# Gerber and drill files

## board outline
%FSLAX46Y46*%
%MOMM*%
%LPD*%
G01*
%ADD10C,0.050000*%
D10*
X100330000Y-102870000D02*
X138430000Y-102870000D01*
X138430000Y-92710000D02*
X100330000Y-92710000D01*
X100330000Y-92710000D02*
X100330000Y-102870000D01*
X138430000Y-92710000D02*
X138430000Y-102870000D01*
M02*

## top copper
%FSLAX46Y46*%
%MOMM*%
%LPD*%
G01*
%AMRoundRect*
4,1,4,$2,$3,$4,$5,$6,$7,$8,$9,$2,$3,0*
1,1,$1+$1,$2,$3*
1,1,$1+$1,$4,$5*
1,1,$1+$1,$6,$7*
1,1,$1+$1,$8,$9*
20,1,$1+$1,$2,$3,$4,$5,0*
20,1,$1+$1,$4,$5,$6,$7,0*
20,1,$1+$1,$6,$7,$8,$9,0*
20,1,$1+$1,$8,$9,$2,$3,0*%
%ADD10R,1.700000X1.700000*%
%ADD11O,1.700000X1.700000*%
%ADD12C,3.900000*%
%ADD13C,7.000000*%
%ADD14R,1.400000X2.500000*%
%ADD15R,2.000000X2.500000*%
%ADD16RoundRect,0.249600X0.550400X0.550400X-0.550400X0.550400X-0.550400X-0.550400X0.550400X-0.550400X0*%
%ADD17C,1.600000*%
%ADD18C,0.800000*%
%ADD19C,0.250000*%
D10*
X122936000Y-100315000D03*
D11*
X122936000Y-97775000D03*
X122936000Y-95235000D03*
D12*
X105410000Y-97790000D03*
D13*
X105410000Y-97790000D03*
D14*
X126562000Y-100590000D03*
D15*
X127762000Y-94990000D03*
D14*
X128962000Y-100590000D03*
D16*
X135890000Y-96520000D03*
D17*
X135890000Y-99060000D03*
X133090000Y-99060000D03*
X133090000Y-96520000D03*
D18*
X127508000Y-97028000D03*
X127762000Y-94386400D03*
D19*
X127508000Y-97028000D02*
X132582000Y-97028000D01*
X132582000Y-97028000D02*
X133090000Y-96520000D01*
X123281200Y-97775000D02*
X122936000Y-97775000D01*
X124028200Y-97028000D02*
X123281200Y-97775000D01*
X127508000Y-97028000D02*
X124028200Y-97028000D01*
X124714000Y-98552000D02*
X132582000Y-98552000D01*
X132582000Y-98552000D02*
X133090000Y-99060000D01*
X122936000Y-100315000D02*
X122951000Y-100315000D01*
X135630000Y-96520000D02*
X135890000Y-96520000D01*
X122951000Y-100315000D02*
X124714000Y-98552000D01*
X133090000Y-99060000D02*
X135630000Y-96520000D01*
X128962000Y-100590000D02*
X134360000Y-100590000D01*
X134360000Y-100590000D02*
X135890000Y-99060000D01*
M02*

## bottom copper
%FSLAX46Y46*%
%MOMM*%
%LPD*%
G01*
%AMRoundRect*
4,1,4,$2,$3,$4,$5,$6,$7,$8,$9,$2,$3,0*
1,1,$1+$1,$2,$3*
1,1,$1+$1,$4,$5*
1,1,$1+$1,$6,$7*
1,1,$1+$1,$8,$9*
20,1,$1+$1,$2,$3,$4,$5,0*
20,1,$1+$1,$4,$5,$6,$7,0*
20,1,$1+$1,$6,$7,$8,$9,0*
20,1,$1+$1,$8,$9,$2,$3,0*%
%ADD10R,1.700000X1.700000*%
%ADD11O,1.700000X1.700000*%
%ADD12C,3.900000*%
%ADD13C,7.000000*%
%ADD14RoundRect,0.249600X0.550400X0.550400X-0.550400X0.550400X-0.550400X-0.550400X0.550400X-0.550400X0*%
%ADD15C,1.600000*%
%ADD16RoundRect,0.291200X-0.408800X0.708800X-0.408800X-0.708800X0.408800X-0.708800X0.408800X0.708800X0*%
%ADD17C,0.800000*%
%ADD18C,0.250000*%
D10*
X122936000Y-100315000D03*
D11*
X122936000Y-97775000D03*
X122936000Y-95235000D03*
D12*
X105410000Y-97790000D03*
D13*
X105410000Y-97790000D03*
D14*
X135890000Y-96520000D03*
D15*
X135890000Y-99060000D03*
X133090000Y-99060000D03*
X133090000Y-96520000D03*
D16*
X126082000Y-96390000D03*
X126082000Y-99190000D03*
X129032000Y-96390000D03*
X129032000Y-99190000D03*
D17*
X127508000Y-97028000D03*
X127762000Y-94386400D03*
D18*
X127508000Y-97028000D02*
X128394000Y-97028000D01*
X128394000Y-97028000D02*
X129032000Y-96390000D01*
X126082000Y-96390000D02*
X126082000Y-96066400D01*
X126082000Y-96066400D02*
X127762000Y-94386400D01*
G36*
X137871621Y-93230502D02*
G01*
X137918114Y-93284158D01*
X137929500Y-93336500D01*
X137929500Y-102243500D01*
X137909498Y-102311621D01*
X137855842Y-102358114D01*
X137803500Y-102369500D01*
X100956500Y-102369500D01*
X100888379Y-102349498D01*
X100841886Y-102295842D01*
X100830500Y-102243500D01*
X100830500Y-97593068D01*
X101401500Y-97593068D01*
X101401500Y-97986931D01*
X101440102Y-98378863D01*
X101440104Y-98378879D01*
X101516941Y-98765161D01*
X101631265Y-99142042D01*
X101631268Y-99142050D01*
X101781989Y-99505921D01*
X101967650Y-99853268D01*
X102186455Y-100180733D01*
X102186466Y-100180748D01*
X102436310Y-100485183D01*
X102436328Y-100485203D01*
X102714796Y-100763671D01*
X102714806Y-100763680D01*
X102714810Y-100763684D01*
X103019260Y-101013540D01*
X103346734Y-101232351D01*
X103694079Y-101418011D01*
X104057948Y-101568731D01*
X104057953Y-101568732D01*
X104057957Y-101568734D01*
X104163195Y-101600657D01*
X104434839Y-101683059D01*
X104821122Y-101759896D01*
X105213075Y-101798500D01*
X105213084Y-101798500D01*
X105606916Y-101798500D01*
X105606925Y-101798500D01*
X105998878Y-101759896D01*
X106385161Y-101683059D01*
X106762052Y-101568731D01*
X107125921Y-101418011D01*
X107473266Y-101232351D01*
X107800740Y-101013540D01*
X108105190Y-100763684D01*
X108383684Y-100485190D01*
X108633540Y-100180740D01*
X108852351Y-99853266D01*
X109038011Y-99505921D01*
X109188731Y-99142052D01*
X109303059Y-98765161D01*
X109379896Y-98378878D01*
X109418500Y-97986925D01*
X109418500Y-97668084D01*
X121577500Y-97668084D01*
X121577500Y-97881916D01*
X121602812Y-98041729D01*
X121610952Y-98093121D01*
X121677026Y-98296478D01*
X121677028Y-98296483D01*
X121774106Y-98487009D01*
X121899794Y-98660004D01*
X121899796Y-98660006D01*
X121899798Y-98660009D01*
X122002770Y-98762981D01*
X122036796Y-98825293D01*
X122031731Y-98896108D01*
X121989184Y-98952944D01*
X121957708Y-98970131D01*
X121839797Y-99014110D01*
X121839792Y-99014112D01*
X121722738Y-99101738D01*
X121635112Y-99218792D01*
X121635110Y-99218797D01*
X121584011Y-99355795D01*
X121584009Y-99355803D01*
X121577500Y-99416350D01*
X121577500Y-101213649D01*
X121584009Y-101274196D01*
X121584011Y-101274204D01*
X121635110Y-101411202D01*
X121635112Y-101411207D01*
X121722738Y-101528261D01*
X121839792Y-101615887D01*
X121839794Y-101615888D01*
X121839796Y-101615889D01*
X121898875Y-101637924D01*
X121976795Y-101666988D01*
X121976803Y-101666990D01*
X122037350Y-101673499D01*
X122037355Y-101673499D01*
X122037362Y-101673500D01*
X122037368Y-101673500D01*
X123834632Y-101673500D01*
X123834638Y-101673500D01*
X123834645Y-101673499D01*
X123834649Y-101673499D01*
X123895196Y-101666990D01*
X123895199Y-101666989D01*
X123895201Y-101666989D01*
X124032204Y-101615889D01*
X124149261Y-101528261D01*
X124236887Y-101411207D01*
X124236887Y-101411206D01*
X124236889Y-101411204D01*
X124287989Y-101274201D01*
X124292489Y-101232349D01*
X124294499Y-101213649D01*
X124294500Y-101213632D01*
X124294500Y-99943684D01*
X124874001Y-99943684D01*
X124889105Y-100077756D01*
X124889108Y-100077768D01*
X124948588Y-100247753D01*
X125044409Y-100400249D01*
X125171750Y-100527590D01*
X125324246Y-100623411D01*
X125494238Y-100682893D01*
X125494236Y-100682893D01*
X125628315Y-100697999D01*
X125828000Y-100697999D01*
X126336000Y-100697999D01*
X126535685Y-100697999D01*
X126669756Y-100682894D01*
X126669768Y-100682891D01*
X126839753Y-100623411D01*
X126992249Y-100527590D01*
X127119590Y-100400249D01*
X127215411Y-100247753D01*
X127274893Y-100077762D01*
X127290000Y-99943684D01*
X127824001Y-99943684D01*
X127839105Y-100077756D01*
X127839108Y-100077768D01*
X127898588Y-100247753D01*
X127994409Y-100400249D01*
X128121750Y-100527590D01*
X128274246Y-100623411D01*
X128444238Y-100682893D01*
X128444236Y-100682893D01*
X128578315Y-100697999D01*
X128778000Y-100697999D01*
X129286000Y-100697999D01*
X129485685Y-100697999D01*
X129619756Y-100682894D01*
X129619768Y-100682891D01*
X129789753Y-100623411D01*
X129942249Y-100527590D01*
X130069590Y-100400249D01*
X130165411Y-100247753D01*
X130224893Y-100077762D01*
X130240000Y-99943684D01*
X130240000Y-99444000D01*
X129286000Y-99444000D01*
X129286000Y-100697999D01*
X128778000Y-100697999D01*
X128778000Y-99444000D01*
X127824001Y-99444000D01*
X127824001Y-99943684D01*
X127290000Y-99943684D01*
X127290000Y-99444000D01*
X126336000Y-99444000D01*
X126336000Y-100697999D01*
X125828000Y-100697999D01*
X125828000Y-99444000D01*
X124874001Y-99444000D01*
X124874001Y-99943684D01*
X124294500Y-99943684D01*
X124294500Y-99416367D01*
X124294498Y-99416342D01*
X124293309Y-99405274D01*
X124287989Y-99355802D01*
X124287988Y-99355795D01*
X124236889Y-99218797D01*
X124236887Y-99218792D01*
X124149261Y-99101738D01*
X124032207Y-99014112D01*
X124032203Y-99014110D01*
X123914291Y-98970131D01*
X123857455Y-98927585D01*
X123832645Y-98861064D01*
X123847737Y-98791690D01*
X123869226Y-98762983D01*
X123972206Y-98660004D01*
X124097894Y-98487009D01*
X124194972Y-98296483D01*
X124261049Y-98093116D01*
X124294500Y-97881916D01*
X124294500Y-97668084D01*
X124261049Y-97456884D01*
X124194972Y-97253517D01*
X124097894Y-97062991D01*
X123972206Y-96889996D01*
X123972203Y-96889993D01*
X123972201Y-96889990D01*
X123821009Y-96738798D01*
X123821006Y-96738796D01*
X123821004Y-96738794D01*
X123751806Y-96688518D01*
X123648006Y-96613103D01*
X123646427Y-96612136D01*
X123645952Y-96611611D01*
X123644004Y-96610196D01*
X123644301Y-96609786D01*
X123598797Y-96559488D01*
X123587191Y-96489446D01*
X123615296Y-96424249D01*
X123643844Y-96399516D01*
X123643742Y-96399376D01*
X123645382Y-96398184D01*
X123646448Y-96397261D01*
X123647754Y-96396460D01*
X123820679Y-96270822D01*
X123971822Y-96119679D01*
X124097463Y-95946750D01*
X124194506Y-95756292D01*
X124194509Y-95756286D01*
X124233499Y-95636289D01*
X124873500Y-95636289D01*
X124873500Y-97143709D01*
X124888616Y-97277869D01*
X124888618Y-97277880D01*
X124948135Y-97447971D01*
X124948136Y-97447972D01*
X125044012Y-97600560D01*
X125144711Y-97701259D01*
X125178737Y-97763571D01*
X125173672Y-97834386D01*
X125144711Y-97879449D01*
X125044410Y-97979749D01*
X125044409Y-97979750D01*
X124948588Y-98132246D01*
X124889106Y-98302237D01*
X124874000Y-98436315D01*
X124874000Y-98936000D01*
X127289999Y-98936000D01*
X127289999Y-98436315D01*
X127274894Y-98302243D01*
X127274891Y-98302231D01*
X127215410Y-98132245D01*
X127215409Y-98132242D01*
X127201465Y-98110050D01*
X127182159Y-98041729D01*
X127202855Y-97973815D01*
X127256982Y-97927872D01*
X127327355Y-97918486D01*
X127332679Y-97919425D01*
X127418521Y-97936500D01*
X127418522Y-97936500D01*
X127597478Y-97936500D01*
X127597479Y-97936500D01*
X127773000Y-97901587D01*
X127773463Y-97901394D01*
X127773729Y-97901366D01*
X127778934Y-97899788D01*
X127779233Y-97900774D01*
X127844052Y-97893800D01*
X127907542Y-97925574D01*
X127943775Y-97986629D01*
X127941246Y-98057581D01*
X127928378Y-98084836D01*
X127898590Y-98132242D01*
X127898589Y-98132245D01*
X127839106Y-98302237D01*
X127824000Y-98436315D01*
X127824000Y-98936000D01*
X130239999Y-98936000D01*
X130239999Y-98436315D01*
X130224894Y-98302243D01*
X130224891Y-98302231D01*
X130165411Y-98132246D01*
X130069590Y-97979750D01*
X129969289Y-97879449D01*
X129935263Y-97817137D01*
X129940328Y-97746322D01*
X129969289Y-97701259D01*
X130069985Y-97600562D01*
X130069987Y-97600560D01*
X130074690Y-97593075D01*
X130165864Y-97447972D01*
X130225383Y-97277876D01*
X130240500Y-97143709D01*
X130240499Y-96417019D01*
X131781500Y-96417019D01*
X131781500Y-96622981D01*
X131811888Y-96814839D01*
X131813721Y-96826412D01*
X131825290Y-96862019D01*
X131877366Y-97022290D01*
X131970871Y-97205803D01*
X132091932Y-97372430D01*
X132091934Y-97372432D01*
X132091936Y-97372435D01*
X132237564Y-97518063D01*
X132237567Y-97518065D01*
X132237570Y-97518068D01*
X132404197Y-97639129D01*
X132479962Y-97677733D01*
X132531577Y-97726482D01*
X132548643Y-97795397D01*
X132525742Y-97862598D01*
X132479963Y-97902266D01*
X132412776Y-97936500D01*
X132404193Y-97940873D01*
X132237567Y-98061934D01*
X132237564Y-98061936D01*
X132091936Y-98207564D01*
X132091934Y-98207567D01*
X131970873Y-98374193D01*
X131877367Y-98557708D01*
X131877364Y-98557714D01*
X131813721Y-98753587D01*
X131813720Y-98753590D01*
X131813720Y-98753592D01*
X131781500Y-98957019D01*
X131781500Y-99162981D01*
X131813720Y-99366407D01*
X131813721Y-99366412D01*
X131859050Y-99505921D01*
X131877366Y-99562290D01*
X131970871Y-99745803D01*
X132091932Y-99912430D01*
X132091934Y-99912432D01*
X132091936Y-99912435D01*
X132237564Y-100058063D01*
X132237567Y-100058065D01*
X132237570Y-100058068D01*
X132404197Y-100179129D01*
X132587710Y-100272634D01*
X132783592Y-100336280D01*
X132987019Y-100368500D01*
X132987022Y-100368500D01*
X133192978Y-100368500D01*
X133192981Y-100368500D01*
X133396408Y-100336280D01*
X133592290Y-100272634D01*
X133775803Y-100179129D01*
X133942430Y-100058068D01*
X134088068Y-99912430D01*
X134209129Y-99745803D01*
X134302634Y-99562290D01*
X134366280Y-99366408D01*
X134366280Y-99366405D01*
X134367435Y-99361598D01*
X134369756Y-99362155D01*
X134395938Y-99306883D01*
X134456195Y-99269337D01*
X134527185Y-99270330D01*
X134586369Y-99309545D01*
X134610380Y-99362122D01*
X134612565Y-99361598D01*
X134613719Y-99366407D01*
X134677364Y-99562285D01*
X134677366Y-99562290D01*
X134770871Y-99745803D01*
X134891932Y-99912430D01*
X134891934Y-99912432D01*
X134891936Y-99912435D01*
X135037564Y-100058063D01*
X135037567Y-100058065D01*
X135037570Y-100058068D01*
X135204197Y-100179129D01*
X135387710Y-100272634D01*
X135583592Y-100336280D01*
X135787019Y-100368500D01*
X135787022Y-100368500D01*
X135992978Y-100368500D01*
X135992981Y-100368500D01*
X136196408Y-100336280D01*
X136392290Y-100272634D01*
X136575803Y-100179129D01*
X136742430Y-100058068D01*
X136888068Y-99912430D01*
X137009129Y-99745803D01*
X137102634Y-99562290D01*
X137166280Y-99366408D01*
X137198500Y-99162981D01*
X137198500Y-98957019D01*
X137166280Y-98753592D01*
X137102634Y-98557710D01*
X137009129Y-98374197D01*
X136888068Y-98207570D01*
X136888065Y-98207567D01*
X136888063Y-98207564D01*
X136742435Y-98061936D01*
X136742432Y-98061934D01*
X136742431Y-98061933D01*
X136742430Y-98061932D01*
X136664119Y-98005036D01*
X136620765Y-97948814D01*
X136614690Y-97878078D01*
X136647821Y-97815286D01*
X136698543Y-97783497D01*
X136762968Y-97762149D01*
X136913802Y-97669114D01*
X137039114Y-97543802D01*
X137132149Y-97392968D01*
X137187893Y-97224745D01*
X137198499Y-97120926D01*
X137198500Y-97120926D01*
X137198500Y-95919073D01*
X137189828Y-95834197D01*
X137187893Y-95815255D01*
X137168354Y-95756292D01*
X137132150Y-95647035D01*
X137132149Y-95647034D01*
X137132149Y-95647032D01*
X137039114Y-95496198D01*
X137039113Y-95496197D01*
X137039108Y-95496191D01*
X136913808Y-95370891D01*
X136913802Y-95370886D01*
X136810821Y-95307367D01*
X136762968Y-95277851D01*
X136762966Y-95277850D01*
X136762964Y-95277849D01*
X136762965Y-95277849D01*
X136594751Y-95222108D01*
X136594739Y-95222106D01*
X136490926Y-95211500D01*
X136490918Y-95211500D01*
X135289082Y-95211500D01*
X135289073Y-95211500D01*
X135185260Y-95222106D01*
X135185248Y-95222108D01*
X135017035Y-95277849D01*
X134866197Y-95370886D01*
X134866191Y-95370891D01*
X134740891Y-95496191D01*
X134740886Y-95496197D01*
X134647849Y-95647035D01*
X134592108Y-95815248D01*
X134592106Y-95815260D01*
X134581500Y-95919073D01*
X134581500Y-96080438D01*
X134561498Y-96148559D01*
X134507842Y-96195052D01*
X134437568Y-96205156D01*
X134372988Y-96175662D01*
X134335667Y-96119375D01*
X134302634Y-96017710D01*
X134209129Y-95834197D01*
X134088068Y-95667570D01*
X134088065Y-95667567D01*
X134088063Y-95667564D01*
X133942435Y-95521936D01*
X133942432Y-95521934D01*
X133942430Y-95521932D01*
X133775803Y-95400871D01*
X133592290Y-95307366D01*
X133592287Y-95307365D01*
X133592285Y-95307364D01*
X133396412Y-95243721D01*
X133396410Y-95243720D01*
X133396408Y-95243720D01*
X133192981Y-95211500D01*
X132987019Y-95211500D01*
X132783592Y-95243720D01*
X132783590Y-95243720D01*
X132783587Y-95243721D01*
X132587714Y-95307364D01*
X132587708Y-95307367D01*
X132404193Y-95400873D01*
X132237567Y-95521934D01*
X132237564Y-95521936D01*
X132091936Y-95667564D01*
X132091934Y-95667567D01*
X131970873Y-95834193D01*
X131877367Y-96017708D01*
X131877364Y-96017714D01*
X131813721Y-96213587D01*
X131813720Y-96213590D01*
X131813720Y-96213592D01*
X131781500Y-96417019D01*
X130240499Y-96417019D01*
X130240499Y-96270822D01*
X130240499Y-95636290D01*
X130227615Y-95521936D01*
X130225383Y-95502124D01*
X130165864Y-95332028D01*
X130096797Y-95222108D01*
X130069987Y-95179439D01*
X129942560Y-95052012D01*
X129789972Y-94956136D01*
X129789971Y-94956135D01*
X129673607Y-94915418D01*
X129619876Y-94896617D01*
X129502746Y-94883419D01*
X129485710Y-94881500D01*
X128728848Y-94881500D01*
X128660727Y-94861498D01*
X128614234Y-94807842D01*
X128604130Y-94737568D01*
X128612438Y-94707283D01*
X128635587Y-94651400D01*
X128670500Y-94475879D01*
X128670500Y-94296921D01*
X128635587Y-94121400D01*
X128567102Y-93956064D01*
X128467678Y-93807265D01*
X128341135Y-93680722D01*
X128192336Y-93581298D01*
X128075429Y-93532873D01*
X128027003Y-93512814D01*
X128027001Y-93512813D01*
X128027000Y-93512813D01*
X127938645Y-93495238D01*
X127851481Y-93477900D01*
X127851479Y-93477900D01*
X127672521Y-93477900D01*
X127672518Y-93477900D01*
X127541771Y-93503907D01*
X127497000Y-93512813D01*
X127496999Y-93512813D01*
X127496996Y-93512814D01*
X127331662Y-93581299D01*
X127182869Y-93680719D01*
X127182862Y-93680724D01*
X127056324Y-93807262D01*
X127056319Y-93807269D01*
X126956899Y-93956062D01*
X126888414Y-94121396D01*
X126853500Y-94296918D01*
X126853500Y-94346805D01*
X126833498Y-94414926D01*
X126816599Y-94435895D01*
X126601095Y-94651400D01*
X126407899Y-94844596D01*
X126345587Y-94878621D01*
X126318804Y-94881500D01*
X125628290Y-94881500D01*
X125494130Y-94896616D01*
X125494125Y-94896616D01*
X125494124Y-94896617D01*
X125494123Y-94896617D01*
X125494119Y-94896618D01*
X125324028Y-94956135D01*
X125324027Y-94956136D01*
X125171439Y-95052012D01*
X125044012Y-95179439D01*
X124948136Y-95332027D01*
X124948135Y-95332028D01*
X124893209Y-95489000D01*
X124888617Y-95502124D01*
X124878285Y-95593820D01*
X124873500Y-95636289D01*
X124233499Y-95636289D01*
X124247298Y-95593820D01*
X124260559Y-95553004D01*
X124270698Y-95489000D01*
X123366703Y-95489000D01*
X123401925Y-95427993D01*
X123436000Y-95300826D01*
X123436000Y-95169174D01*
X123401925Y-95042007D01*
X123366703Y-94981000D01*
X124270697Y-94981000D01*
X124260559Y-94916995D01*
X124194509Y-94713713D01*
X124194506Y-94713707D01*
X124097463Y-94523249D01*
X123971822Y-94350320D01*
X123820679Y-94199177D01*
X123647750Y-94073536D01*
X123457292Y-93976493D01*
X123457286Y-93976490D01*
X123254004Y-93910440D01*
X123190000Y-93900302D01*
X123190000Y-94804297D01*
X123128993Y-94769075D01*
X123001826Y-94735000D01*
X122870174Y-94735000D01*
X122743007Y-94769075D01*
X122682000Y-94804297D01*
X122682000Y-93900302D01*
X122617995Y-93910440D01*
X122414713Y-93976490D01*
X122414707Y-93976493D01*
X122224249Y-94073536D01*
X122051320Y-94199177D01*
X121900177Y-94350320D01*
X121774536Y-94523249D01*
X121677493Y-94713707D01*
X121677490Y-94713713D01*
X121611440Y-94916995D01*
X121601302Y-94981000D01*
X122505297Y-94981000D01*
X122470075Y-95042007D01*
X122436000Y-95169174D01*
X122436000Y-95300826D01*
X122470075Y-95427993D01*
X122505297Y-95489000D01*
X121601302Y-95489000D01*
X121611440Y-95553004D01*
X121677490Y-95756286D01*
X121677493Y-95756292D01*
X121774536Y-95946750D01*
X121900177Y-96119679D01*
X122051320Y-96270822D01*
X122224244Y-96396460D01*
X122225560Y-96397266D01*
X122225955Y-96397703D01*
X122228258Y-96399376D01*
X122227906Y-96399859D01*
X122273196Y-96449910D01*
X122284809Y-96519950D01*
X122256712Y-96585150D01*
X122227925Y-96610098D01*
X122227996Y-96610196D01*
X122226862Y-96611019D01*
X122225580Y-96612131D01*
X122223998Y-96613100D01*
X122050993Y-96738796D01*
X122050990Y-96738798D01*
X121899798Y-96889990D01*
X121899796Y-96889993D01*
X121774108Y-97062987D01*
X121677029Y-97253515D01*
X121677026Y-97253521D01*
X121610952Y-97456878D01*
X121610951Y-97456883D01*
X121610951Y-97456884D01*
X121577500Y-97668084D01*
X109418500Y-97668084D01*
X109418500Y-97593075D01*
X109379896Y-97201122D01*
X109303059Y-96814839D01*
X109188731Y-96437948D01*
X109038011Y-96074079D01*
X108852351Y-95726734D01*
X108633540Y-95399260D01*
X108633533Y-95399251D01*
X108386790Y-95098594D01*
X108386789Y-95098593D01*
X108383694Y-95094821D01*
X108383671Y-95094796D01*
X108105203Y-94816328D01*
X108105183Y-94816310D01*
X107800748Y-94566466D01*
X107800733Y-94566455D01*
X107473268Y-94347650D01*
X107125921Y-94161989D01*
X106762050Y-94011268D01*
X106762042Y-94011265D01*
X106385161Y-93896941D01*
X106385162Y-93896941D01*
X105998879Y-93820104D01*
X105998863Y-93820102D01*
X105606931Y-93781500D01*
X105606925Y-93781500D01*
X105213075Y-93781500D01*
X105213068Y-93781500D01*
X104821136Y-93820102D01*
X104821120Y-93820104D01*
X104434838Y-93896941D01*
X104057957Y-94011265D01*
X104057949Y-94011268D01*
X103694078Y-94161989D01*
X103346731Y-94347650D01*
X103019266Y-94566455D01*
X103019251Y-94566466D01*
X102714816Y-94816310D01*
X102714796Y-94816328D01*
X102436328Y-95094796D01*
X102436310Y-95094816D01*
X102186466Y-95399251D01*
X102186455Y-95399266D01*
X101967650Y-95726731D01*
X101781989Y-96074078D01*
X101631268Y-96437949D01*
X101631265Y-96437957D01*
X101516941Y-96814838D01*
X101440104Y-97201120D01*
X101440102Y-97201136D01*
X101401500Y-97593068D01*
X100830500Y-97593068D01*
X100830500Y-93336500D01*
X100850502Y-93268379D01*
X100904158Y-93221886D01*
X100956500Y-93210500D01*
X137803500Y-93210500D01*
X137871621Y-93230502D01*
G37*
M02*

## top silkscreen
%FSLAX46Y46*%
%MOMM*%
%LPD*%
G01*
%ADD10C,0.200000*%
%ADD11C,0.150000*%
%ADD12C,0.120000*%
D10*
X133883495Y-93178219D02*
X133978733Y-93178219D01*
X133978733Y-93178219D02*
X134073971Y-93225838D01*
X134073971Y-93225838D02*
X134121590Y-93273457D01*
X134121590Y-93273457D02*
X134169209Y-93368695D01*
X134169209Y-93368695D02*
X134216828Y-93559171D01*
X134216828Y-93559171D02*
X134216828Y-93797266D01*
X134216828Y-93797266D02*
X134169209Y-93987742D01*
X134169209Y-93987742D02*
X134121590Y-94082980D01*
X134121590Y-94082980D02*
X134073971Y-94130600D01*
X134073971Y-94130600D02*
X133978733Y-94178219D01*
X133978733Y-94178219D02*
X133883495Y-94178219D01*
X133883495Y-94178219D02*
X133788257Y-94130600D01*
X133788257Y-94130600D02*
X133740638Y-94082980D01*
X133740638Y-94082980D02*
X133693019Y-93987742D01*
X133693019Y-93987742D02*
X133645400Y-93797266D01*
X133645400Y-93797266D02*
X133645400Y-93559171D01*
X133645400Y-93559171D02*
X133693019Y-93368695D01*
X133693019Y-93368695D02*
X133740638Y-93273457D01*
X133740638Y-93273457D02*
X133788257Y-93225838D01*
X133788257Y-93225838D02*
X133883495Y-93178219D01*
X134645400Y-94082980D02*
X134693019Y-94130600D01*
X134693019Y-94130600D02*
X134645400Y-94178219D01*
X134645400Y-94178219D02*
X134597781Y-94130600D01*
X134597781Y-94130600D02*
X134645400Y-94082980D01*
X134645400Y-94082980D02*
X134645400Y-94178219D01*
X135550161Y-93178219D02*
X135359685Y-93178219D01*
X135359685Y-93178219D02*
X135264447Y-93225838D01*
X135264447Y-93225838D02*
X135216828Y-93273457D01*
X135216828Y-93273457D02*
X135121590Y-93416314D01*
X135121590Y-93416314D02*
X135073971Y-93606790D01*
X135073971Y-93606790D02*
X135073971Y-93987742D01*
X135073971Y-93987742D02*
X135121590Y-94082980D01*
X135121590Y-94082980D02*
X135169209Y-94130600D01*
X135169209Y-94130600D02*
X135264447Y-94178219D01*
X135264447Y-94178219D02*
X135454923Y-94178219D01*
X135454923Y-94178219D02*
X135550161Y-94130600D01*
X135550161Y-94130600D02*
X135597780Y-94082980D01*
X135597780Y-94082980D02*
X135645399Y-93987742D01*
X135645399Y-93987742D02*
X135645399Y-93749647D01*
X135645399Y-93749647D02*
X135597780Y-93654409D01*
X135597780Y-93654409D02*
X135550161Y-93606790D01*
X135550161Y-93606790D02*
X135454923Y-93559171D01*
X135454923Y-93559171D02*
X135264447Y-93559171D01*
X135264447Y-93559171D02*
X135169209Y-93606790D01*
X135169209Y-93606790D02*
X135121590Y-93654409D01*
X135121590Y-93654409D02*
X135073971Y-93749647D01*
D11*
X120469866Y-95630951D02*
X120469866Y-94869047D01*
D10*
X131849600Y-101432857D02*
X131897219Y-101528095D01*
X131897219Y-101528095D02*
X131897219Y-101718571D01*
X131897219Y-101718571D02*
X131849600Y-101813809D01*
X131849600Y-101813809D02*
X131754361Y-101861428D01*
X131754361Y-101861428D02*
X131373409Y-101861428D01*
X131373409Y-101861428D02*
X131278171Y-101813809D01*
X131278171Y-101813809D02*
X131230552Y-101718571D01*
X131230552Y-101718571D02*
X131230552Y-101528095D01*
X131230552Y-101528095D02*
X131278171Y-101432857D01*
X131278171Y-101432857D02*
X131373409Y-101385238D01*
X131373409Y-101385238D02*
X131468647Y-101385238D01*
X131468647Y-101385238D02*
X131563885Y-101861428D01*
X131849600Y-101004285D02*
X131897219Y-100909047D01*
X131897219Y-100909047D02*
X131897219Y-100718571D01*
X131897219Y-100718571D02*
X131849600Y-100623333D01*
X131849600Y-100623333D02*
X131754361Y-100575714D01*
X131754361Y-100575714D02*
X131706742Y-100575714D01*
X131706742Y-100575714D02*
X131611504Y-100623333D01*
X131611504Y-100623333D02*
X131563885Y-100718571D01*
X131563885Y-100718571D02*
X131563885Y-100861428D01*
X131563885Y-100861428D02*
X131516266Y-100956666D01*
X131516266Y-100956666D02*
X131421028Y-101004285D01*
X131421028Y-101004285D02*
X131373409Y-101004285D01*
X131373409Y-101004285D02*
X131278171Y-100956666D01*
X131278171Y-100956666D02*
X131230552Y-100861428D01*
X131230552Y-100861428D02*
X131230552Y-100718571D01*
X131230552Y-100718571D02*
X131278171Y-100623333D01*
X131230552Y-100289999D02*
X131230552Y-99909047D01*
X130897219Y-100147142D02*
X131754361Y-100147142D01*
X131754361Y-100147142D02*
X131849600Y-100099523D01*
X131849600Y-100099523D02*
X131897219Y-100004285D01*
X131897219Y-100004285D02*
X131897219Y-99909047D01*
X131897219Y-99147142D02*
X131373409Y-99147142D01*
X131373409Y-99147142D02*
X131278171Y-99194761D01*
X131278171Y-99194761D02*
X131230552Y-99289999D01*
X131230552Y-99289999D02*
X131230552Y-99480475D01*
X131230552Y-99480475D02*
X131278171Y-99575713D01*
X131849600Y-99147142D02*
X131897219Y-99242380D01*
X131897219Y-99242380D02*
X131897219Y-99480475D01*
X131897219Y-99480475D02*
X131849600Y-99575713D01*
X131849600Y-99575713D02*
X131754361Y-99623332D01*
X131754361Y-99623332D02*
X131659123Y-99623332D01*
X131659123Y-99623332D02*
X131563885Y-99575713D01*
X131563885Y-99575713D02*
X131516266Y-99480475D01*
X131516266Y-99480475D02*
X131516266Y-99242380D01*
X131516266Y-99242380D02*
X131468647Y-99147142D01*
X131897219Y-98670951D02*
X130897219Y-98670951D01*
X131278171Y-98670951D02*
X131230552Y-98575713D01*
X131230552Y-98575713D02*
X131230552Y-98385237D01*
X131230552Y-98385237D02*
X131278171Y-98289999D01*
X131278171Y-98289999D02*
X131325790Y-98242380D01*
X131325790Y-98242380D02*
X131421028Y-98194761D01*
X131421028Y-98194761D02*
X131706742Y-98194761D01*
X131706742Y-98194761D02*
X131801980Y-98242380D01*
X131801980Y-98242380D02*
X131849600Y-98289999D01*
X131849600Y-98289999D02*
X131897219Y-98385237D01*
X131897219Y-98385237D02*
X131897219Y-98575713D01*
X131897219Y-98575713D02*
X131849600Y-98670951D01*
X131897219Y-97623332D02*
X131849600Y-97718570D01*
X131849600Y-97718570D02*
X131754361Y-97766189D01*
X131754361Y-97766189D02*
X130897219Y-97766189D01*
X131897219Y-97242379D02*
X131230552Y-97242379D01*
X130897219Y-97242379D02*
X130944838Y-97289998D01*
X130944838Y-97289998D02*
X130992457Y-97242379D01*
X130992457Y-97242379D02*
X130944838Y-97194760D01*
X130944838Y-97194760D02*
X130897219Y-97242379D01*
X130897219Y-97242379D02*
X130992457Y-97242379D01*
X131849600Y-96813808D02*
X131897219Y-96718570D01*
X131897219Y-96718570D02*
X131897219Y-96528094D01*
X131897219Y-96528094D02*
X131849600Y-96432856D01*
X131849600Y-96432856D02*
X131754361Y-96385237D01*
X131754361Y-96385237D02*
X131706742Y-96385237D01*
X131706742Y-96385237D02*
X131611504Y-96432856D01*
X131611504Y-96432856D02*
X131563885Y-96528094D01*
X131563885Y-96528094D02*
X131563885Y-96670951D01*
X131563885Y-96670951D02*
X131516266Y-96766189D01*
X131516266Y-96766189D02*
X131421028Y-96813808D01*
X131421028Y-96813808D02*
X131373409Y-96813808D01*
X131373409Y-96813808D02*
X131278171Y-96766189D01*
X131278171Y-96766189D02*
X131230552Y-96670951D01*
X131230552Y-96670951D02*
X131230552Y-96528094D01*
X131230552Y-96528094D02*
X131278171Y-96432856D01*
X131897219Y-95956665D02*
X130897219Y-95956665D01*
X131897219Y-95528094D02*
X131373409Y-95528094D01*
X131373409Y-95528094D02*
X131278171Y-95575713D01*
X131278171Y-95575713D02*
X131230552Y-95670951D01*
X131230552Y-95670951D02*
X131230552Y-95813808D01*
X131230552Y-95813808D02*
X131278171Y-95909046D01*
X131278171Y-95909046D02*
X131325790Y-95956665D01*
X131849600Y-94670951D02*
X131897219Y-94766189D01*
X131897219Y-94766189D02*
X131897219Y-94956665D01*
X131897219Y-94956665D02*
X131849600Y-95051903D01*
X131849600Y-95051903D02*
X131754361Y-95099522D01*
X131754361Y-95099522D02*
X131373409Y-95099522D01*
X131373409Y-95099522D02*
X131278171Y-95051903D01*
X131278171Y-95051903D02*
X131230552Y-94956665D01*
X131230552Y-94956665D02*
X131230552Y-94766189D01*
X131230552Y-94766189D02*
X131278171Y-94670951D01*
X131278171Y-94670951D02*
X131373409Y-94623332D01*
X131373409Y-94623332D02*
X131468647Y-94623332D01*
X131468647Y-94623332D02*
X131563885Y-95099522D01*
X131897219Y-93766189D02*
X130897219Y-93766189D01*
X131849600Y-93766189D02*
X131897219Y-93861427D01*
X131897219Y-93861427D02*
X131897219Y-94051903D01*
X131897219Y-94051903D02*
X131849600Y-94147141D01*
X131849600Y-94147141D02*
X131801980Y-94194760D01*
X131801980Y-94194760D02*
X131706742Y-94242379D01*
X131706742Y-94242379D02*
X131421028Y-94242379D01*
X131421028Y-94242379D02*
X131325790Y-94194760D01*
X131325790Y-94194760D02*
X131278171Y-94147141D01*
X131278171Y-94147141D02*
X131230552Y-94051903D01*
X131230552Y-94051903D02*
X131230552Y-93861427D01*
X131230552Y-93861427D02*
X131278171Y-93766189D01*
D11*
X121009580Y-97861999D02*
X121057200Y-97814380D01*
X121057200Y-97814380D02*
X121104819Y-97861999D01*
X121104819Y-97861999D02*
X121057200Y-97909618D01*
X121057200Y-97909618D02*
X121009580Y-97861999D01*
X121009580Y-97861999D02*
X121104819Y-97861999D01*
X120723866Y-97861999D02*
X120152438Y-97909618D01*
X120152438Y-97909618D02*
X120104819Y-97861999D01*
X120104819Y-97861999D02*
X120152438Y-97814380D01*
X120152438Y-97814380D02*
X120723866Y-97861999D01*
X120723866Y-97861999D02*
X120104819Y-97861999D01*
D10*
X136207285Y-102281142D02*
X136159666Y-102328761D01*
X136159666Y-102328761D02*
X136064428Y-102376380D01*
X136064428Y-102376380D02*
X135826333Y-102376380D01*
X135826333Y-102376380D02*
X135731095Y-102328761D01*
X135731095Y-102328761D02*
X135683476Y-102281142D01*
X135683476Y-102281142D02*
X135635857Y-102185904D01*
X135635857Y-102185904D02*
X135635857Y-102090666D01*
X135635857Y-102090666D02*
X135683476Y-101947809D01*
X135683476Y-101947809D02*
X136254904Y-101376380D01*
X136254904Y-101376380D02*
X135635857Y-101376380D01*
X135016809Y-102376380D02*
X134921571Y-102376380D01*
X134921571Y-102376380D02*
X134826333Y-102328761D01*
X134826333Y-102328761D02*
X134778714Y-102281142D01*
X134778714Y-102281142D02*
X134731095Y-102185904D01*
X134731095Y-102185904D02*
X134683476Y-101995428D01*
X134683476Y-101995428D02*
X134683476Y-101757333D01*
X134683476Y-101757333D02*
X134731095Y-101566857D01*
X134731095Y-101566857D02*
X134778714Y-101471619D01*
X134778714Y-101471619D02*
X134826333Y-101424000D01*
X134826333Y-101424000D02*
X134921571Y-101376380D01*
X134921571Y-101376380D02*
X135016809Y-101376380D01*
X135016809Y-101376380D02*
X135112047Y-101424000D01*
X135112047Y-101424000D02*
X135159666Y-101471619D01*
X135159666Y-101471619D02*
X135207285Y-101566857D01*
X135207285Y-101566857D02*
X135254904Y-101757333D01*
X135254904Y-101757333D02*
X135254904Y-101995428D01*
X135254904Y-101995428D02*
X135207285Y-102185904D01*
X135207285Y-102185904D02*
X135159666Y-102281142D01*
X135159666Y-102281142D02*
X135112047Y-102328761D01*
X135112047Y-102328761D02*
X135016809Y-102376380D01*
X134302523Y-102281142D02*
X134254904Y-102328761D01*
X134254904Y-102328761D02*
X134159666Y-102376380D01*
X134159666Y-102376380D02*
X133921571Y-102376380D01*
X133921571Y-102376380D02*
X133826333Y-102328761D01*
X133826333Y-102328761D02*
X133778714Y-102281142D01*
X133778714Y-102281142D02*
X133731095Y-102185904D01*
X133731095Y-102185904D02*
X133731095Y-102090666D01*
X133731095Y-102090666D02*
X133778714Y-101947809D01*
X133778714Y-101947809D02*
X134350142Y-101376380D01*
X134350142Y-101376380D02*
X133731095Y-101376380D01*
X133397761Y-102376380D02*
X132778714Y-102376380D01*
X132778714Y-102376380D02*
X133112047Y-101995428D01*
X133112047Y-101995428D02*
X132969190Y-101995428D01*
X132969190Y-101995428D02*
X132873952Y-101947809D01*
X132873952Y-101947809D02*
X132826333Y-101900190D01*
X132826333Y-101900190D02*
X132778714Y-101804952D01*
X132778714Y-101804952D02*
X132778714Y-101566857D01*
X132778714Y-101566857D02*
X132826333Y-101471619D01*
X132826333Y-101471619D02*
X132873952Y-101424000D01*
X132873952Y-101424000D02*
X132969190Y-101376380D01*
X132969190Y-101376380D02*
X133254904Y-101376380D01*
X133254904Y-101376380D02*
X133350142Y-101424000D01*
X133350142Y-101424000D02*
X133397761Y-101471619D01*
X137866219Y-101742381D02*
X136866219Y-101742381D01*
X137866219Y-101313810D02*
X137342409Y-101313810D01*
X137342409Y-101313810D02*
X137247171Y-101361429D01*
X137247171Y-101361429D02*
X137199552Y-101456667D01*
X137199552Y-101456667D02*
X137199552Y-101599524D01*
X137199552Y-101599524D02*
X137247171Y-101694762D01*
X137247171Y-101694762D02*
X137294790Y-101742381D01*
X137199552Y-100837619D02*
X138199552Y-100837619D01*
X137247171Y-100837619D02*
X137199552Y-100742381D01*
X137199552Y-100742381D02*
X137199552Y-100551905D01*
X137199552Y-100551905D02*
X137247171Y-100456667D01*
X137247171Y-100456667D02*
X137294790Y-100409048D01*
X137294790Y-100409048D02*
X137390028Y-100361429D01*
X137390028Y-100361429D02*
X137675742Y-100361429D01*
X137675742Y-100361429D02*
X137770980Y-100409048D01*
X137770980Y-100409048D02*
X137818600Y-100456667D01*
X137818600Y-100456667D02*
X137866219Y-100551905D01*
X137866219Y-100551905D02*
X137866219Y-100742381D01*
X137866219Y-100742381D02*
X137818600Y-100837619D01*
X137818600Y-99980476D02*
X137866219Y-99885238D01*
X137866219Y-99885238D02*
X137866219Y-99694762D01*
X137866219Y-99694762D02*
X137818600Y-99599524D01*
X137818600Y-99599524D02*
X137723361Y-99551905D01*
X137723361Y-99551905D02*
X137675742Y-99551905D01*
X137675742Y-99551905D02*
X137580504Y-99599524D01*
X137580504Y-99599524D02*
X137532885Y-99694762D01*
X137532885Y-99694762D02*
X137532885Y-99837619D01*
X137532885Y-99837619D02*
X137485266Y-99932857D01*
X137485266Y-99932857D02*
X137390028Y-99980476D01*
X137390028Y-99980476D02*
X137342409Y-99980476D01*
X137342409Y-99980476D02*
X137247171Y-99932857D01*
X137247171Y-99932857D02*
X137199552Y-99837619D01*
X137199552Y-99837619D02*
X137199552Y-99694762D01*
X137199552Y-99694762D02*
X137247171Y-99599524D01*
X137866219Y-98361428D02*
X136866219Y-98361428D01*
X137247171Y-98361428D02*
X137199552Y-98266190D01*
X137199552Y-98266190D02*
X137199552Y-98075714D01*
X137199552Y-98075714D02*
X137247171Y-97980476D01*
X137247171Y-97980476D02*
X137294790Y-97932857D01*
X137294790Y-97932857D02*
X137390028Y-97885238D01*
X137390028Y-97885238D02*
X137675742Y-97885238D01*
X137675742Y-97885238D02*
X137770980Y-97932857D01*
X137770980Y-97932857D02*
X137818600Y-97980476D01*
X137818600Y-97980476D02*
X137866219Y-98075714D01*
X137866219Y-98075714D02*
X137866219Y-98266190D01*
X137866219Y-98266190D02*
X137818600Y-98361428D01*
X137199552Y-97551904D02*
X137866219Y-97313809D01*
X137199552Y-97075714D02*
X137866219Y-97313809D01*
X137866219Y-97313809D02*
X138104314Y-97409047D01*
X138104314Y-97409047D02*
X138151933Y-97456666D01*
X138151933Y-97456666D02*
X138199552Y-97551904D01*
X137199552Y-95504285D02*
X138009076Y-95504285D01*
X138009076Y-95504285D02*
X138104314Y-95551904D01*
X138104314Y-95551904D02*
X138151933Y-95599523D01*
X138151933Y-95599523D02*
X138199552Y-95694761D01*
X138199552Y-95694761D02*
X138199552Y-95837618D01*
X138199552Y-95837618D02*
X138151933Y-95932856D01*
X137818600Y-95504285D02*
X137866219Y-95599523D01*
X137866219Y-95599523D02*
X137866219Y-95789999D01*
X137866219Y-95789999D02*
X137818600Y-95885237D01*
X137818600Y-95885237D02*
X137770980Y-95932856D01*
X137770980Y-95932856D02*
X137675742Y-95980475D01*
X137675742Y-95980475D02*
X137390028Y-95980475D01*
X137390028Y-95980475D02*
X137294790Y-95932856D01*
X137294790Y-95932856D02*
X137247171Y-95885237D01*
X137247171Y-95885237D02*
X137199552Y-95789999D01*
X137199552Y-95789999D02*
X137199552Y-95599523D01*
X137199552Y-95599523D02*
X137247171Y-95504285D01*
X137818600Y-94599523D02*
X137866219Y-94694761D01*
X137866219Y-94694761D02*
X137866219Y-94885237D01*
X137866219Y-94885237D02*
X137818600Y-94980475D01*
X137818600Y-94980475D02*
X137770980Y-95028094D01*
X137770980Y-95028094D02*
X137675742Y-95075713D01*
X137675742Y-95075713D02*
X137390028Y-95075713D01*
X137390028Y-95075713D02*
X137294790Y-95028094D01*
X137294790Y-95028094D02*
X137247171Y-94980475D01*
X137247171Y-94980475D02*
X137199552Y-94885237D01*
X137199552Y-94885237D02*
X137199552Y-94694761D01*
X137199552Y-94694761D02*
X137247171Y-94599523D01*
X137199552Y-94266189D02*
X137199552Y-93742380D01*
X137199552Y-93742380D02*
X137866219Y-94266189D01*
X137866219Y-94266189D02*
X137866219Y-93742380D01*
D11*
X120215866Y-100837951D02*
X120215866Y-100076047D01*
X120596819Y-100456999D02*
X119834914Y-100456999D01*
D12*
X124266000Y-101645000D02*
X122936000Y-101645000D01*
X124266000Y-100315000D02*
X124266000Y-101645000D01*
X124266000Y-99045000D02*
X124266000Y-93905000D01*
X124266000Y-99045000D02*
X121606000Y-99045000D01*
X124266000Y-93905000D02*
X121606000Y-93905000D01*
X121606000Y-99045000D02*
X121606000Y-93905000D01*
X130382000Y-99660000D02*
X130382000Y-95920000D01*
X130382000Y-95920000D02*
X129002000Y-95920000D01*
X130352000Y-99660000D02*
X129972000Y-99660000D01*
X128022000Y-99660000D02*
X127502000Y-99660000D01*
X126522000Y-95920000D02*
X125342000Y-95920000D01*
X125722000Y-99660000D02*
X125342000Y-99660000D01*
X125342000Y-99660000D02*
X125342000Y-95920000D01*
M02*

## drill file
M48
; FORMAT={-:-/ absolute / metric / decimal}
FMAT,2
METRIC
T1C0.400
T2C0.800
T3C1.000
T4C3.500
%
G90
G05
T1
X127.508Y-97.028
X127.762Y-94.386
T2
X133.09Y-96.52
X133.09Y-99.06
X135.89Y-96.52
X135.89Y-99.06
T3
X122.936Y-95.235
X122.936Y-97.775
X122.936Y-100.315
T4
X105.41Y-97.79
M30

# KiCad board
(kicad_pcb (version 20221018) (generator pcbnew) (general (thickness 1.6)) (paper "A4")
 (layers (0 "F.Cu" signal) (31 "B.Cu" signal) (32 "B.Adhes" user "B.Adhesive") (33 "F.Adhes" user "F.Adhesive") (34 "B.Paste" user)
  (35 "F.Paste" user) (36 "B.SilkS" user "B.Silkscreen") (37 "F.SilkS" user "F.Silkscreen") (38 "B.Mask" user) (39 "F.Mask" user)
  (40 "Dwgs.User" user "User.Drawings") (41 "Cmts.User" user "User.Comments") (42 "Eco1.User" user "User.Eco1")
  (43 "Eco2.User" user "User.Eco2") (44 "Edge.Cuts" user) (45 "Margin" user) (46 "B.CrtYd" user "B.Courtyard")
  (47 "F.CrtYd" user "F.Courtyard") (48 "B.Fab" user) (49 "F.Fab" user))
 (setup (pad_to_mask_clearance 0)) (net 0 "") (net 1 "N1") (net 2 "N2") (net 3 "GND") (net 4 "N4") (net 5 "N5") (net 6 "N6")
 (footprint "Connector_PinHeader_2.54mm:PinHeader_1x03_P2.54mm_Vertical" (layer "F.Cu") (at 122.936 100.315 180)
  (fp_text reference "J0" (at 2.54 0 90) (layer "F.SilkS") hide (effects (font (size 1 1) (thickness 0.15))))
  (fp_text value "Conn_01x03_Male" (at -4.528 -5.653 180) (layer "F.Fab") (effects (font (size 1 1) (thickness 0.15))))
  (fp_line (start -1.33 -1.33) (end 0 -1.33) (stroke (width 0.12) (type solid)) (layer "F.SilkS"))
  (fp_line (start -1.33 0) (end -1.33 -1.33) (stroke (width 0.12) (type solid)) (layer "F.SilkS"))
  (fp_line (start -1.33 1.27) (end -1.33 6.41) (stroke (width 0.12) (type solid)) (layer "F.SilkS"))
  (fp_line (start -1.33 1.27) (end 1.33 1.27) (stroke (width 0.12) (type solid)) (layer "F.SilkS"))
  (fp_line (start -1.33 6.41) (end 1.33 6.41) (stroke (width 0.12) (type solid)) (layer "F.SilkS"))
  (fp_line (start 1.33 1.27) (end 1.33 6.41) (stroke (width 0.12) (type solid)) (layer "F.SilkS"))
  (pad "1" thru_hole rect (at 0 0 180) (size 1.7 1.7) (drill 1) (layers "*.Cu" "*.Mask") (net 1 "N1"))
  (pad "2" thru_hole oval (at 0 2.54 180) (size 1.7 1.7) (drill 1) (layers "*.Cu" "*.Mask") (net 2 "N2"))
  (pad "3" thru_hole oval (at 0 5.08 180) (size 1.7 1.7) (drill 1) (layers "*.Cu" "*.Mask") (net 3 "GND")))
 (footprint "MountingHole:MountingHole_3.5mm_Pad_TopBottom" (layer "F.Cu") (at 105.41 97.79)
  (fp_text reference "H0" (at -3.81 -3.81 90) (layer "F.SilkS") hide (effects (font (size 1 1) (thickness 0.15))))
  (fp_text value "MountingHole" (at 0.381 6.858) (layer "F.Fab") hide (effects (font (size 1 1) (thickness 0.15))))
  (pad "1" thru_hole circle (at 0 0) (size 3.9 3.9) (drill 3.5) (layers "*.Cu" "*.Mask"))
  (pad "1" connect circle (at 0 0) (size 7 7) (layers "F.Cu" "F.Mask"))
  (pad "1" connect circle (at 0 0) (size 7 7) (layers "B.Cu" "B.Mask")))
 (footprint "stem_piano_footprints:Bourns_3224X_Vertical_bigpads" (layer "F.Cu") (at 127.762 97.79 180)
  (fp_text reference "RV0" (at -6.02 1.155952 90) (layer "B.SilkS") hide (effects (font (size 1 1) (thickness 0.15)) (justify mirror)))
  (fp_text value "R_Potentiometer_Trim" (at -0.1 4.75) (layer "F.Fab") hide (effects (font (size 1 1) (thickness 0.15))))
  (fp_line (start -2.62 -1.87) (end -2.62 1.87) (stroke (width 0.12) (type solid)) (layer "F.SilkS"))
  (fp_line (start -2.62 1.87) (end -1.24 1.87) (stroke (width 0.12) (type solid)) (layer "F.SilkS"))
  (fp_line (start -2.59 -1.87) (end -2.21 -1.87) (stroke (width 0.12) (type solid)) (layer "F.SilkS"))
  (fp_line (start -0.26 -1.87) (end 0.26 -1.87) (stroke (width 0.12) (type solid)) (layer "F.SilkS"))
  (fp_line (start 1.24 1.87) (end 2.42 1.87) (stroke (width 0.12) (type solid)) (layer "F.SilkS"))
  (fp_line (start 2.04 -1.87) (end 2.42 -1.87) (stroke (width 0.12) (type solid)) (layer "F.SilkS"))
  (fp_line (start 2.42 -1.87) (end 2.42 1.87) (stroke (width 0.12) (type solid)) (layer "F.SilkS"))
  (pad "1" smd rect (at 1.2 -2.8 180) (size 1.4 2.5) (layers "F.Cu" "F.Paste" "F.Mask") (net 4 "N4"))
  (pad "2" smd rect (at 0 2.8 180) (size 2 2.5) (layers "F.Cu" "F.Paste" "F.Mask") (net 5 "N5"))
  (pad "3" smd rect (at -1.2 -2.8 180) (size 1.4 2.5) (layers "F.Cu" "F.Paste" "F.Mask") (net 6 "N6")))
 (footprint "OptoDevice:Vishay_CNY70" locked (layer "B.Cu") (at 135.89 96.52 180)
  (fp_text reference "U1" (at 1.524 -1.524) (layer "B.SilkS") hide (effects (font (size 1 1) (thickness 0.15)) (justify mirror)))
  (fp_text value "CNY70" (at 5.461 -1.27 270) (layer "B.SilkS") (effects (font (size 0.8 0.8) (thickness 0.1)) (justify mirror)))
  (pad "1" thru_hole roundrect locked (at 0 0 180) (size 1.6 1.6) (drill 0.8) (layers "*.Cu" "*.Mask") (roundrect_rratio 0.156) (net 1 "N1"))
  (pad "2" thru_hole circle locked (at 0 -2.54 180) (size 1.6 1.6) (drill 0.8) (layers "*.Cu" "*.Mask") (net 6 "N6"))
  (pad "3" thru_hole circle locked (at 2.8 -2.54 180) (size 1.6 1.6) (drill 0.8) (layers "*.Cu" "*.Mask") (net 1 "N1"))
  (pad "4" thru_hole circle locked (at 2.8 0 180) (size 1.6 1.6) (drill 0.8) (layers "*.Cu" "*.Mask") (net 2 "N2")))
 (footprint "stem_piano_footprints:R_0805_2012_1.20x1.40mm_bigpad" (layer "B.Cu") (at 126.082 97.79 -90)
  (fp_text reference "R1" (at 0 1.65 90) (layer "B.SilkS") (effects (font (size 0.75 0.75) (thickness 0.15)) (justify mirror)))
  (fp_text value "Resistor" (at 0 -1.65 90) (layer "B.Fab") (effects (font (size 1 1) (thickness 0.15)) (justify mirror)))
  (pad "1" smd roundrect (at -1.4 0 270) (size 2 1.4) (layers "B.Cu" "B.Paste" "B.Mask") (roundrect_rratio 0.208) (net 5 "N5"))
  (pad "2" smd roundrect (at 1.4 0 270) (size 2 1.4) (layers "B.Cu" "B.Paste" "B.Mask") (roundrect_rratio 0.208) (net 3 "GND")))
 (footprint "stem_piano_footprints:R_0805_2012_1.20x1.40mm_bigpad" (layer "B.Cu") (at 129.032 97.79 -90)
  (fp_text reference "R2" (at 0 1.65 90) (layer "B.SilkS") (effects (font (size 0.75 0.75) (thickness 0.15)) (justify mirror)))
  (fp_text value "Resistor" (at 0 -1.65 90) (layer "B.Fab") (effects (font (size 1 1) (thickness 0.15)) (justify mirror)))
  (pad "1" smd roundrect (at -1.4 0 270) (size 2 1.4) (layers "B.Cu" "B.Paste" "B.Mask") (roundrect_rratio 0.208) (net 2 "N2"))
  (pad "2" smd roundrect (at 1.4 0 270) (size 2 1.4) (layers "B.Cu" "B.Paste" "B.Mask") (roundrect_rratio 0.208) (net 3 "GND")))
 (gr_line (start 100.33 102.87) (end 138.43 102.87) (stroke (width 0.05) (type solid)) (layer "Edge.Cuts"))
 (gr_line (start 138.43 92.71) (end 100.33 92.71) (stroke (width 0.05) (type solid)) (layer "Edge.Cuts"))
 (gr_line (start 100.33 92.71) (end 100.33 102.87) (stroke (width 0.05) (type solid)) (layer "Edge.Cuts"))
 (gr_line (start 138.43 92.71) (end 138.43 102.87) (stroke (width 0.05) (type solid)) (layer "Edge.Cuts"))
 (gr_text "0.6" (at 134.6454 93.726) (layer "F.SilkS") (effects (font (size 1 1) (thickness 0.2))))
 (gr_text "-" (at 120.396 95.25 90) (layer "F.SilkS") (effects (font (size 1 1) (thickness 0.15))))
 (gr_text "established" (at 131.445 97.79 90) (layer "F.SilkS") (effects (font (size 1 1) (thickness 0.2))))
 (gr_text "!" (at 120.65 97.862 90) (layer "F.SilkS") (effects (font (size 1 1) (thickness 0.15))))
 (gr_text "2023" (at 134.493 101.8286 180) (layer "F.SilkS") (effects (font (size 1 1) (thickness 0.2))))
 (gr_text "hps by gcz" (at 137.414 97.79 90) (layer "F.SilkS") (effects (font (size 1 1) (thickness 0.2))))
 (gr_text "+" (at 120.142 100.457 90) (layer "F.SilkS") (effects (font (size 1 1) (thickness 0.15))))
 (segment (start 127.508 97.028) (end 132.582 97.028) (width 0.25) (layer "F.Cu") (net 2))
 (segment (start 132.582 97.028) (end 133.09 96.52) (width 0.25) (layer "F.Cu") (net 2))
 (segment (start 123.2812 97.775) (end 122.936 97.775) (width 0.25) (layer "F.Cu") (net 2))
 (segment (start 124.0282 97.028) (end 123.2812 97.775) (width 0.25) (layer "F.Cu") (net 2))
 (segment (start 127.508 97.028) (end 124.0282 97.028) (width 0.25) (layer "F.Cu") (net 2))
 (via (at 127.508 97.028) (size 0.8) (drill 0.4) (layers "F.Cu" "B.Cu") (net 2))
 (segment (start 127.508 97.028) (end 128.394 97.028) (width 0.25) (layer "B.Cu") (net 2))
 (segment (start 128.394 97.028) (end 129.032 96.39) (width 0.25) (layer "B.Cu") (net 2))
 (segment (start 124.714 98.552) (end 132.582 98.552) (width 0.25) (layer "F.Cu") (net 1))
 (segment (start 132.582 98.552) (end 133.09 99.06) (width 0.25) (layer "F.Cu") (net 1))
 (segment (start 122.936 100.315) (end 122.951 100.315) (width 0.25) (layer "F.Cu") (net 1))
 (segment (start 135.63 96.52) (end 135.89 96.52) (width 0.25) (layer "F.Cu") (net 1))
 (segment (start 122.951 100.315) (end 124.714 98.552) (width 0.25) (layer "F.Cu") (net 1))
 (segment (start 133.09 99.06) (end 135.63 96.52) (width 0.25) (layer "F.Cu") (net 1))
 (via (at 127.762 94.3864) (size 0.8) (drill 0.4) (layers "F.Cu" "B.Cu") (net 5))
 (segment (start 126.082 96.39) (end 126.082 96.0664) (width 0.25) (layer "B.Cu") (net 5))
 (segment (start 126.082 96.0664) (end 127.762 94.3864) (width 0.25) (layer "B.Cu") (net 5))
 (segment (start 128.962 100.59) (end 134.36 100.59) (width 0.25) (layer "F.Cu") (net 6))
 (segment (start 134.36 100.59) (end 135.89 99.06) (width 0.25) (layer "F.Cu") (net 6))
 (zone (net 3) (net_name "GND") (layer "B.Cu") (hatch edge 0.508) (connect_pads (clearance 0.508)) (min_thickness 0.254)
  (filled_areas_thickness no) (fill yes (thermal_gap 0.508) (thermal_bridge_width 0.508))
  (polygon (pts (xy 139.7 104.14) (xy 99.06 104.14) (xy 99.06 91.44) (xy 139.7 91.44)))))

